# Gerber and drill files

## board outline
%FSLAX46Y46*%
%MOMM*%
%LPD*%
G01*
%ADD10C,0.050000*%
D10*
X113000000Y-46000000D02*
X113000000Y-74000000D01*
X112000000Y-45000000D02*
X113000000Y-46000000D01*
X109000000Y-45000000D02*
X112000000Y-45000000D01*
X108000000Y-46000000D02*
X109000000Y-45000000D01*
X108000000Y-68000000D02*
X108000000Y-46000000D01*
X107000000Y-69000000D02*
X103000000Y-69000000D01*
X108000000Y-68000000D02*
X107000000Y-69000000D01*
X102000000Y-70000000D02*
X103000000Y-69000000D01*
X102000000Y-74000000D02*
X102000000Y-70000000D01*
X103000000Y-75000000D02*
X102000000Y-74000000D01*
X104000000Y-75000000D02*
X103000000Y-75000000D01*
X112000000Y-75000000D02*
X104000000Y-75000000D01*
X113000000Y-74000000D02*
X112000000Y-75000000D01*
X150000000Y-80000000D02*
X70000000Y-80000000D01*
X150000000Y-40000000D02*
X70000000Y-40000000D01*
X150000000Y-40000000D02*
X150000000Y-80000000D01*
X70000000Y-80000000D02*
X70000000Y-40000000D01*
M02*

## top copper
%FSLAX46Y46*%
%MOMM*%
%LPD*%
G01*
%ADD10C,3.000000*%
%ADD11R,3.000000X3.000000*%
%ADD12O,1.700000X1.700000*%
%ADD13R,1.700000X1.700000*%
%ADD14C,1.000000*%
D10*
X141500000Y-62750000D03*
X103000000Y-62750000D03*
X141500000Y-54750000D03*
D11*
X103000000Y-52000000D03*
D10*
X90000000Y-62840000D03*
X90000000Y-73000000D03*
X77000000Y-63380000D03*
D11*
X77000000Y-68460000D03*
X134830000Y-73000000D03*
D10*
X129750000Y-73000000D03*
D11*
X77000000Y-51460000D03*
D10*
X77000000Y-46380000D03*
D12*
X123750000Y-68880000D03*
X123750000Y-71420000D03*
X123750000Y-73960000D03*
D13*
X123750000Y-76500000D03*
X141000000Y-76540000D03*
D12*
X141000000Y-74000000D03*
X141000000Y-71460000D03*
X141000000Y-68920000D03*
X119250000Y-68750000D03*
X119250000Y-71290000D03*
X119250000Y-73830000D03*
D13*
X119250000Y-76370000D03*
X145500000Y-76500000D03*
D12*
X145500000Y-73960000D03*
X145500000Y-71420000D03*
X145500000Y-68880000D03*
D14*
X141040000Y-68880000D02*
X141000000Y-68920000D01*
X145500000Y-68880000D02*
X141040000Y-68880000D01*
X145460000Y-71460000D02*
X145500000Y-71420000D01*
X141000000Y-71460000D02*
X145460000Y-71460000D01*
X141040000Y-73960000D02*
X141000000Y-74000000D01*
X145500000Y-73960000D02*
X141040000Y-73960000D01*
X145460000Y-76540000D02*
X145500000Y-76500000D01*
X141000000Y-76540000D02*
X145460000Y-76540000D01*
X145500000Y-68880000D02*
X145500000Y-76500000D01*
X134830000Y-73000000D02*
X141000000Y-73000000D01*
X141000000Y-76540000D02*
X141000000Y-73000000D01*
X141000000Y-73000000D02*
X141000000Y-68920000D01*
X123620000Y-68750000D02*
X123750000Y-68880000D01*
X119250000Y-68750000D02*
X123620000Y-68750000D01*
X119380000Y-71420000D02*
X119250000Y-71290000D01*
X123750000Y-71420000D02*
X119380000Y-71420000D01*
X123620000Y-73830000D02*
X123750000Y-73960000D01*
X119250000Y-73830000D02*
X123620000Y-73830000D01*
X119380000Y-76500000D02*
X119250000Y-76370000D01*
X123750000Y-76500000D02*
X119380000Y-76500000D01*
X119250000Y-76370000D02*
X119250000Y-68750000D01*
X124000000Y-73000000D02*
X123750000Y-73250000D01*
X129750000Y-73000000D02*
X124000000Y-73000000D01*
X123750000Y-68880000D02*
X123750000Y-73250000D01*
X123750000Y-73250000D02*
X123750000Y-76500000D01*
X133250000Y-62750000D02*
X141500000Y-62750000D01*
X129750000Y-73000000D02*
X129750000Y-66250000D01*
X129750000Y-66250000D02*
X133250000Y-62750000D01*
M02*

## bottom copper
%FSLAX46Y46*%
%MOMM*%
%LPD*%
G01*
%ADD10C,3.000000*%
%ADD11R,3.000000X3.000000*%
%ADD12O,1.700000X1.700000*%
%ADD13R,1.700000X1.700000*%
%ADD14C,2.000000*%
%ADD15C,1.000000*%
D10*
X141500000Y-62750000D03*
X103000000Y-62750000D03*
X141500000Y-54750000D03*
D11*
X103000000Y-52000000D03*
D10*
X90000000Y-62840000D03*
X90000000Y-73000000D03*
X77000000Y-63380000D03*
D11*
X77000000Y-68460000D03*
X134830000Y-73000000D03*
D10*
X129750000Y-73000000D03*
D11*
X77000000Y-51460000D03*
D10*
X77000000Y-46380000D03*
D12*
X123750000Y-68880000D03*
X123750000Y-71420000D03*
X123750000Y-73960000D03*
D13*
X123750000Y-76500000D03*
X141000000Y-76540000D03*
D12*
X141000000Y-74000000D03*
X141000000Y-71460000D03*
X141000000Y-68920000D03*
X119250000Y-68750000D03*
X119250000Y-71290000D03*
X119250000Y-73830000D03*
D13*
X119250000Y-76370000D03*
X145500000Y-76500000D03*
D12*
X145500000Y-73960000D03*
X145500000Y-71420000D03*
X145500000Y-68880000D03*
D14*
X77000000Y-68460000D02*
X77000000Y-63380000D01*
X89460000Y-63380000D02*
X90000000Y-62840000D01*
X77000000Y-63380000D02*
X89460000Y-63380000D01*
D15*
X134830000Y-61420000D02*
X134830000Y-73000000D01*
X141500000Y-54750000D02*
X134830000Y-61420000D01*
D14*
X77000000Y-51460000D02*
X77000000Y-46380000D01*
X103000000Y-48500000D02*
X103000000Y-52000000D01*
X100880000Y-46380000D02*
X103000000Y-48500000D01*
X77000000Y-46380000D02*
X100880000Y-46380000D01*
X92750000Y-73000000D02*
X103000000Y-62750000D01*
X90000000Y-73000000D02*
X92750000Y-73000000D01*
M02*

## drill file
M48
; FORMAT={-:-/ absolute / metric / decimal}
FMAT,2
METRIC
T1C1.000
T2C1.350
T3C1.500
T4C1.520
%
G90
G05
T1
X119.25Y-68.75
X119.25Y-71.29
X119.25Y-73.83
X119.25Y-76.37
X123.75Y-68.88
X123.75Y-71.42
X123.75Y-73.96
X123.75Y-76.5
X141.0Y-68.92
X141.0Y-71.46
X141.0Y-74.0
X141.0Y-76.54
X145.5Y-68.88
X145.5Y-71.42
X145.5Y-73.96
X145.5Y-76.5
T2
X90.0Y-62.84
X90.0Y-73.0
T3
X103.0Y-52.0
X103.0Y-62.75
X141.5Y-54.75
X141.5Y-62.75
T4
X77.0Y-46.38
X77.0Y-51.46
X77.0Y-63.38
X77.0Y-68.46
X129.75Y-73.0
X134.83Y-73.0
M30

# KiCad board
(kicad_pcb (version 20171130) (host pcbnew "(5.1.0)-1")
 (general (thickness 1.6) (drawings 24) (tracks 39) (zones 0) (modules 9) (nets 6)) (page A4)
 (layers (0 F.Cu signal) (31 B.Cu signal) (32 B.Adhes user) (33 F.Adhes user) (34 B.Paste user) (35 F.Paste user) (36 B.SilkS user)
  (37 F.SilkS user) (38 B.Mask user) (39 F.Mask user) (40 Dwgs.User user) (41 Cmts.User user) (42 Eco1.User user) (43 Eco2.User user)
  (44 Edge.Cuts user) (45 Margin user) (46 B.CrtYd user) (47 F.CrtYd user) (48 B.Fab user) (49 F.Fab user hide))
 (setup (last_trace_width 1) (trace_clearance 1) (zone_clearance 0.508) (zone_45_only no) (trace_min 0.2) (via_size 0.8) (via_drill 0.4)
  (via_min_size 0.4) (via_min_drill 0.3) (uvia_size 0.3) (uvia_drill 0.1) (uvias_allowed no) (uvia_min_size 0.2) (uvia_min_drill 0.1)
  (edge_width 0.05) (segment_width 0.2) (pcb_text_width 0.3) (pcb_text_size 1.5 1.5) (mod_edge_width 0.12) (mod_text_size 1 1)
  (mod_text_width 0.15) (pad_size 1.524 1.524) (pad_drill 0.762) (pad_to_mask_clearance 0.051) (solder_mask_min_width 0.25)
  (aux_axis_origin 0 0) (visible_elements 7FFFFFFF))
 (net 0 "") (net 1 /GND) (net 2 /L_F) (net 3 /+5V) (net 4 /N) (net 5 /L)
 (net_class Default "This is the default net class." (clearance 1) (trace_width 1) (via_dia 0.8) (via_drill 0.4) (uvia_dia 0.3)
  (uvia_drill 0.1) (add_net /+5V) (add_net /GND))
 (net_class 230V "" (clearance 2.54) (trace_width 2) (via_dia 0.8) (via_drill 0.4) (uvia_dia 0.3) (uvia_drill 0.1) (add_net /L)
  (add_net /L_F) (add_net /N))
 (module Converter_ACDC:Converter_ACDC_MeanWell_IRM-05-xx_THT (layer F.Cu) (at 103 52)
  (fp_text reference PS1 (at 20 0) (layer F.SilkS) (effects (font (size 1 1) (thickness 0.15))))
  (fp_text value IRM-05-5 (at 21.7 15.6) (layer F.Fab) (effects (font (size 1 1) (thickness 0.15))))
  (pad 3 thru_hole circle (at 38.5 10.75) (size 3 3) (drill 1.5) (layers *.Cu *.Mask) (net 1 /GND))
  (pad 2 thru_hole circle (at 0 10.75) (size 3 3) (drill 1.5) (layers *.Cu *.Mask) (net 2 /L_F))
  (pad 4 thru_hole circle (at 38.5 2.75) (size 3 3) (drill 1.5) (layers *.Cu *.Mask) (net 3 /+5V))
  (pad 1 thru_hole rect (at 0 0) (size 3 3) (drill 1.5) (layers *.Cu *.Mask) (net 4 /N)))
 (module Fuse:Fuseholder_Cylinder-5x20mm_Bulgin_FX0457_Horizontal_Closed (layer F.Cu) (at 90 73 90)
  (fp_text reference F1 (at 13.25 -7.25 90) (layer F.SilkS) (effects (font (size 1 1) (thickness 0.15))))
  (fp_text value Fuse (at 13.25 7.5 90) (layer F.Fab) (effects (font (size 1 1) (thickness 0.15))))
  (pad 2 thru_hole circle (at 10.16 0 90) (size 3 3) (drill 1.35) (layers *.Cu *.Mask) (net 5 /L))
  (pad 1 thru_hole circle (at 0 0 90) (size 3 3) (drill 1.35) (layers *.Cu *.Mask) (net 2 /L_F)))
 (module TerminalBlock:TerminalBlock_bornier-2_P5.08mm (layer F.Cu) (at 77 68.46 90)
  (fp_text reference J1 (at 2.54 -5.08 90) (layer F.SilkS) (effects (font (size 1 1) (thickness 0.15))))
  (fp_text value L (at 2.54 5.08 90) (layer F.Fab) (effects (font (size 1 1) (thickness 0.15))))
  (pad 2 thru_hole circle (at 5.08 0 90) (size 3 3) (drill 1.52) (layers *.Cu *.Mask) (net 5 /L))
  (pad 1 thru_hole rect (at 0 0 90) (size 3 3) (drill 1.52) (layers *.Cu *.Mask) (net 5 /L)))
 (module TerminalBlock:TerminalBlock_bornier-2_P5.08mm (layer F.Cu) (at 134.83 73 180)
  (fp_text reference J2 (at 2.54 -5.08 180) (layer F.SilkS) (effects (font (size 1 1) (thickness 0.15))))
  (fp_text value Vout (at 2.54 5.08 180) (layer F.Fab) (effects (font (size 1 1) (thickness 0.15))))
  (pad 1 thru_hole rect (at 0 0 180) (size 3 3) (drill 1.52) (layers *.Cu *.Mask) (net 3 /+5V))
  (pad 2 thru_hole circle (at 5.08 0 180) (size 3 3) (drill 1.52) (layers *.Cu *.Mask) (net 1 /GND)))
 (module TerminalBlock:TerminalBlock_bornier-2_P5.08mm (layer F.Cu) (at 77 51.46 90)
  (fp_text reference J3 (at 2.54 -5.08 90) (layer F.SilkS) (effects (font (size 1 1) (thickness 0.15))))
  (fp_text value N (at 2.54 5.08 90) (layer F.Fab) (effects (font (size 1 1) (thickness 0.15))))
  (pad 1 thru_hole rect (at 0 0 90) (size 3 3) (drill 1.52) (layers *.Cu *.Mask) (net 4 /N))
  (pad 2 thru_hole circle (at 5.08 0 90) (size 3 3) (drill 1.52) (layers *.Cu *.Mask) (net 4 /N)))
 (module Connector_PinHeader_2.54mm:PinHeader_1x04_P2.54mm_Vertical (layer F.Cu) (at 123.75 76.5 180)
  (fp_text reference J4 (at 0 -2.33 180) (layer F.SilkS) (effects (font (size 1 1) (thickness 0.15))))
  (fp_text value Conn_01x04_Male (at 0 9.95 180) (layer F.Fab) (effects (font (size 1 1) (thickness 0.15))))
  (pad 4 thru_hole oval (at 0 7.62 180) (size 1.7 1.7) (drill 1) (layers *.Cu *.Mask) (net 1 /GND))
  (pad 3 thru_hole oval (at 0 5.08 180) (size 1.7 1.7) (drill 1) (layers *.Cu *.Mask) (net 1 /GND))
  (pad 2 thru_hole oval (at 0 2.54 180) (size 1.7 1.7) (drill 1) (layers *.Cu *.Mask) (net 1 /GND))
  (pad 1 thru_hole rect (at 0 0 180) (size 1.7 1.7) (drill 1) (layers *.Cu *.Mask) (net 1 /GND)))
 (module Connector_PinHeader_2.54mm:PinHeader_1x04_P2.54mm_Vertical (layer F.Cu) (at 141 76.54 180)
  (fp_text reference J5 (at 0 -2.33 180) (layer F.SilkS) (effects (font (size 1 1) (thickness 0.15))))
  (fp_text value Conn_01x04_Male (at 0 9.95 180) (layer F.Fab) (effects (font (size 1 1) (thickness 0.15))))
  (pad 1 thru_hole rect (at 0 0 180) (size 1.7 1.7) (drill 1) (layers *.Cu *.Mask) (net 3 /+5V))
  (pad 2 thru_hole oval (at 0 2.54 180) (size 1.7 1.7) (drill 1) (layers *.Cu *.Mask) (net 3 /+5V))
  (pad 3 thru_hole oval (at 0 5.08 180) (size 1.7 1.7) (drill 1) (layers *.Cu *.Mask) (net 3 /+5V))
  (pad 4 thru_hole oval (at 0 7.62 180) (size 1.7 1.7) (drill 1) (layers *.Cu *.Mask) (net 3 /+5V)))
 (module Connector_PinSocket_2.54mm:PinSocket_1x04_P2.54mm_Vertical (layer F.Cu) (at 119.25 76.37 180)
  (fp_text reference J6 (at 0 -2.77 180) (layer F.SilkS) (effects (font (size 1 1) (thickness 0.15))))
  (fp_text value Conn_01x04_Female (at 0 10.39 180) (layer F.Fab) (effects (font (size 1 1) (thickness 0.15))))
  (pad 4 thru_hole oval (at 0 7.62 180) (size 1.7 1.7) (drill 1) (layers *.Cu *.Mask) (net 1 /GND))
  (pad 3 thru_hole oval (at 0 5.08 180) (size 1.7 1.7) (drill 1) (layers *.Cu *.Mask) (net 1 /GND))
  (pad 2 thru_hole oval (at 0 2.54 180) (size 1.7 1.7) (drill 1) (layers *.Cu *.Mask) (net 1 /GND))
  (pad 1 thru_hole rect (at 0 0 180) (size 1.7 1.7) (drill 1) (layers *.Cu *.Mask) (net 1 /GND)))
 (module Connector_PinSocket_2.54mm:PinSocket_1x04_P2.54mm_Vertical (layer F.Cu) (at 145.5 76.5 180)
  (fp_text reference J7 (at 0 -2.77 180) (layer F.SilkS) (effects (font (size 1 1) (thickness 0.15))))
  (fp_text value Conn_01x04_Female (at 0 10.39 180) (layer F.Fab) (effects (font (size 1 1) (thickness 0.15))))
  (pad 1 thru_hole rect (at 0 0 180) (size 1.7 1.7) (drill 1) (layers *.Cu *.Mask) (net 3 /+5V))
  (pad 2 thru_hole oval (at 0 2.54 180) (size 1.7 1.7) (drill 1) (layers *.Cu *.Mask) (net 3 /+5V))
  (pad 3 thru_hole oval (at 0 5.08 180) (size 1.7 1.7) (drill 1) (layers *.Cu *.Mask) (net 3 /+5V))
  (pad 4 thru_hole oval (at 0 7.62 180) (size 1.7 1.7) (drill 1) (layers *.Cu *.Mask) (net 3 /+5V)))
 (gr_line (start 113 46) (end 113 74) (layer Edge.Cuts) (width 0.05))
 (gr_line (start 112 45) (end 113 46) (layer Edge.Cuts) (width 0.05))
 (gr_line (start 109 45) (end 112 45) (layer Edge.Cuts) (width 0.05))
 (gr_line (start 108 46) (end 109 45) (layer Edge.Cuts) (width 0.05))
 (gr_line (start 108 68) (end 108 46) (layer Edge.Cuts) (width 0.05))
 (gr_line (start 107 69) (end 103 69) (layer Edge.Cuts) (width 0.05))
 (gr_line (start 108 68) (end 107 69) (layer Edge.Cuts) (width 0.05))
 (gr_line (start 102 70) (end 103 69) (layer Edge.Cuts) (width 0.05))
 (gr_line (start 102 74) (end 102 70) (layer Edge.Cuts) (width 0.05))
 (gr_line (start 103 75) (end 102 74) (layer Edge.Cuts) (width 0.05))
 (gr_line (start 104 75) (end 103 75) (layer Edge.Cuts) (width 0.05))
 (gr_line (start 112 75) (end 104 75) (layer Edge.Cuts) (width 0.05))
 (gr_line (start 113 74) (end 112 75) (layer Edge.Cuts) (width 0.05))
 (gr_line (start 150 80) (end 70 80) (layer Edge.Cuts) (width 0.05))
 (gr_line (start 150 40) (end 70 40) (layer Edge.Cuts) (width 0.05))
 (gr_line (start 150 40) (end 150 80) (layer Edge.Cuts) (width 0.05))
 (gr_line (start 70 80) (end 70 40) (layer Edge.Cuts) (width 0.05))
 (segment (start 77 68.46) (end 77 63.38) (width 2) (layer B.Cu) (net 5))
 (segment (start 89.46 63.38) (end 90 62.84) (width 2) (layer B.Cu) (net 5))
 (segment (start 77 63.38) (end 89.46 63.38) (width 2) (layer B.Cu) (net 5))
 (segment (start 141.04 68.88) (end 141 68.92) (width 1) (layer F.Cu) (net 3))
 (segment (start 145.5 68.88) (end 141.04 68.88) (width 1) (layer F.Cu) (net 3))
 (segment (start 145.46 71.46) (end 145.5 71.42) (width 1) (layer F.Cu) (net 3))
 (segment (start 141 71.46) (end 145.46 71.46) (width 1) (layer F.Cu) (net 3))
 (segment (start 141.04 73.96) (end 141 74) (width 1) (layer F.Cu) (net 3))
 (segment (start 145.5 73.96) (end 141.04 73.96) (width 1) (layer F.Cu) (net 3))
 (segment (start 145.46 76.54) (end 145.5 76.5) (width 1) (layer F.Cu) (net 3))
 (segment (start 141 76.54) (end 145.46 76.54) (width 1) (layer F.Cu) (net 3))
 (segment (start 145.5 68.88) (end 145.5 76.5) (width 1) (layer F.Cu) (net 3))
 (segment (start 134.83 73) (end 141 73) (width 1) (layer F.Cu) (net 3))
 (segment (start 141 76.54) (end 141 73) (width 1) (layer F.Cu) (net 3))
 (segment (start 141 73) (end 141 68.92) (width 1) (layer F.Cu) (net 3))
 (segment (start 134.83 61.42) (end 134.83 73) (width 1) (layer B.Cu) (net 3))
 (segment (start 141.5 54.75) (end 134.83 61.42) (width 1) (layer B.Cu) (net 3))
 (segment (start 123.62 68.75) (end 123.75 68.88) (width 1) (layer F.Cu) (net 1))
 (segment (start 119.25 68.75) (end 123.62 68.75) (width 1) (layer F.Cu) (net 1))
 (segment (start 119.38 71.42) (end 119.25 71.29) (width 1) (layer F.Cu) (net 1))
 (segment (start 123.75 71.42) (end 119.38 71.42) (width 1) (layer F.Cu) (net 1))
 (segment (start 123.62 73.83) (end 123.75 73.96) (width 1) (layer F.Cu) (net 1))
 (segment (start 119.25 73.83) (end 123.62 73.83) (width 1) (layer F.Cu) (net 1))
 (segment (start 119.38 76.5) (end 119.25 76.37) (width 1) (layer F.Cu) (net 1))
 (segment (start 123.75 76.5) (end 119.38 76.5) (width 1) (layer F.Cu) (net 1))
 (segment (start 119.25 76.37) (end 119.25 68.75) (width 1) (layer F.Cu) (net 1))
 (segment (start 124 73) (end 123.75 73.25) (width 1) (layer F.Cu) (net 1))
 (segment (start 129.75 73) (end 124 73) (width 1) (layer F.Cu) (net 1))
 (segment (start 123.75 68.88) (end 123.75 73.25) (width 1) (layer F.Cu) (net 1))
 (segment (start 123.75 73.25) (end 123.75 76.5) (width 1) (layer F.Cu) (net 1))
 (segment (start 133.25 62.75) (end 141.5 62.75) (width 1) (layer F.Cu) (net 1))
 (segment (start 129.75 73) (end 129.75 66.25) (width 1) (layer F.Cu) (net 1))
 (segment (start 129.75 66.25) (end 133.25 62.75) (width 1) (layer F.Cu) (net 1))
 (segment (start 77 51.46) (end 77 46.38) (width 2) (layer B.Cu) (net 4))
 (segment (start 103 48.5) (end 103 52) (width 2) (layer B.Cu) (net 4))
 (segment (start 100.88 46.38) (end 103 48.5) (width 2) (layer B.Cu) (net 4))
 (segment (start 77 46.38) (end 100.88 46.38) (width 2) (layer B.Cu) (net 4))
 (segment (start 92.75 73) (end 103 62.75) (width 2) (layer B.Cu) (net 2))
 (segment (start 90 73) (end 92.75 73) (width 2) (layer B.Cu) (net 2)))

